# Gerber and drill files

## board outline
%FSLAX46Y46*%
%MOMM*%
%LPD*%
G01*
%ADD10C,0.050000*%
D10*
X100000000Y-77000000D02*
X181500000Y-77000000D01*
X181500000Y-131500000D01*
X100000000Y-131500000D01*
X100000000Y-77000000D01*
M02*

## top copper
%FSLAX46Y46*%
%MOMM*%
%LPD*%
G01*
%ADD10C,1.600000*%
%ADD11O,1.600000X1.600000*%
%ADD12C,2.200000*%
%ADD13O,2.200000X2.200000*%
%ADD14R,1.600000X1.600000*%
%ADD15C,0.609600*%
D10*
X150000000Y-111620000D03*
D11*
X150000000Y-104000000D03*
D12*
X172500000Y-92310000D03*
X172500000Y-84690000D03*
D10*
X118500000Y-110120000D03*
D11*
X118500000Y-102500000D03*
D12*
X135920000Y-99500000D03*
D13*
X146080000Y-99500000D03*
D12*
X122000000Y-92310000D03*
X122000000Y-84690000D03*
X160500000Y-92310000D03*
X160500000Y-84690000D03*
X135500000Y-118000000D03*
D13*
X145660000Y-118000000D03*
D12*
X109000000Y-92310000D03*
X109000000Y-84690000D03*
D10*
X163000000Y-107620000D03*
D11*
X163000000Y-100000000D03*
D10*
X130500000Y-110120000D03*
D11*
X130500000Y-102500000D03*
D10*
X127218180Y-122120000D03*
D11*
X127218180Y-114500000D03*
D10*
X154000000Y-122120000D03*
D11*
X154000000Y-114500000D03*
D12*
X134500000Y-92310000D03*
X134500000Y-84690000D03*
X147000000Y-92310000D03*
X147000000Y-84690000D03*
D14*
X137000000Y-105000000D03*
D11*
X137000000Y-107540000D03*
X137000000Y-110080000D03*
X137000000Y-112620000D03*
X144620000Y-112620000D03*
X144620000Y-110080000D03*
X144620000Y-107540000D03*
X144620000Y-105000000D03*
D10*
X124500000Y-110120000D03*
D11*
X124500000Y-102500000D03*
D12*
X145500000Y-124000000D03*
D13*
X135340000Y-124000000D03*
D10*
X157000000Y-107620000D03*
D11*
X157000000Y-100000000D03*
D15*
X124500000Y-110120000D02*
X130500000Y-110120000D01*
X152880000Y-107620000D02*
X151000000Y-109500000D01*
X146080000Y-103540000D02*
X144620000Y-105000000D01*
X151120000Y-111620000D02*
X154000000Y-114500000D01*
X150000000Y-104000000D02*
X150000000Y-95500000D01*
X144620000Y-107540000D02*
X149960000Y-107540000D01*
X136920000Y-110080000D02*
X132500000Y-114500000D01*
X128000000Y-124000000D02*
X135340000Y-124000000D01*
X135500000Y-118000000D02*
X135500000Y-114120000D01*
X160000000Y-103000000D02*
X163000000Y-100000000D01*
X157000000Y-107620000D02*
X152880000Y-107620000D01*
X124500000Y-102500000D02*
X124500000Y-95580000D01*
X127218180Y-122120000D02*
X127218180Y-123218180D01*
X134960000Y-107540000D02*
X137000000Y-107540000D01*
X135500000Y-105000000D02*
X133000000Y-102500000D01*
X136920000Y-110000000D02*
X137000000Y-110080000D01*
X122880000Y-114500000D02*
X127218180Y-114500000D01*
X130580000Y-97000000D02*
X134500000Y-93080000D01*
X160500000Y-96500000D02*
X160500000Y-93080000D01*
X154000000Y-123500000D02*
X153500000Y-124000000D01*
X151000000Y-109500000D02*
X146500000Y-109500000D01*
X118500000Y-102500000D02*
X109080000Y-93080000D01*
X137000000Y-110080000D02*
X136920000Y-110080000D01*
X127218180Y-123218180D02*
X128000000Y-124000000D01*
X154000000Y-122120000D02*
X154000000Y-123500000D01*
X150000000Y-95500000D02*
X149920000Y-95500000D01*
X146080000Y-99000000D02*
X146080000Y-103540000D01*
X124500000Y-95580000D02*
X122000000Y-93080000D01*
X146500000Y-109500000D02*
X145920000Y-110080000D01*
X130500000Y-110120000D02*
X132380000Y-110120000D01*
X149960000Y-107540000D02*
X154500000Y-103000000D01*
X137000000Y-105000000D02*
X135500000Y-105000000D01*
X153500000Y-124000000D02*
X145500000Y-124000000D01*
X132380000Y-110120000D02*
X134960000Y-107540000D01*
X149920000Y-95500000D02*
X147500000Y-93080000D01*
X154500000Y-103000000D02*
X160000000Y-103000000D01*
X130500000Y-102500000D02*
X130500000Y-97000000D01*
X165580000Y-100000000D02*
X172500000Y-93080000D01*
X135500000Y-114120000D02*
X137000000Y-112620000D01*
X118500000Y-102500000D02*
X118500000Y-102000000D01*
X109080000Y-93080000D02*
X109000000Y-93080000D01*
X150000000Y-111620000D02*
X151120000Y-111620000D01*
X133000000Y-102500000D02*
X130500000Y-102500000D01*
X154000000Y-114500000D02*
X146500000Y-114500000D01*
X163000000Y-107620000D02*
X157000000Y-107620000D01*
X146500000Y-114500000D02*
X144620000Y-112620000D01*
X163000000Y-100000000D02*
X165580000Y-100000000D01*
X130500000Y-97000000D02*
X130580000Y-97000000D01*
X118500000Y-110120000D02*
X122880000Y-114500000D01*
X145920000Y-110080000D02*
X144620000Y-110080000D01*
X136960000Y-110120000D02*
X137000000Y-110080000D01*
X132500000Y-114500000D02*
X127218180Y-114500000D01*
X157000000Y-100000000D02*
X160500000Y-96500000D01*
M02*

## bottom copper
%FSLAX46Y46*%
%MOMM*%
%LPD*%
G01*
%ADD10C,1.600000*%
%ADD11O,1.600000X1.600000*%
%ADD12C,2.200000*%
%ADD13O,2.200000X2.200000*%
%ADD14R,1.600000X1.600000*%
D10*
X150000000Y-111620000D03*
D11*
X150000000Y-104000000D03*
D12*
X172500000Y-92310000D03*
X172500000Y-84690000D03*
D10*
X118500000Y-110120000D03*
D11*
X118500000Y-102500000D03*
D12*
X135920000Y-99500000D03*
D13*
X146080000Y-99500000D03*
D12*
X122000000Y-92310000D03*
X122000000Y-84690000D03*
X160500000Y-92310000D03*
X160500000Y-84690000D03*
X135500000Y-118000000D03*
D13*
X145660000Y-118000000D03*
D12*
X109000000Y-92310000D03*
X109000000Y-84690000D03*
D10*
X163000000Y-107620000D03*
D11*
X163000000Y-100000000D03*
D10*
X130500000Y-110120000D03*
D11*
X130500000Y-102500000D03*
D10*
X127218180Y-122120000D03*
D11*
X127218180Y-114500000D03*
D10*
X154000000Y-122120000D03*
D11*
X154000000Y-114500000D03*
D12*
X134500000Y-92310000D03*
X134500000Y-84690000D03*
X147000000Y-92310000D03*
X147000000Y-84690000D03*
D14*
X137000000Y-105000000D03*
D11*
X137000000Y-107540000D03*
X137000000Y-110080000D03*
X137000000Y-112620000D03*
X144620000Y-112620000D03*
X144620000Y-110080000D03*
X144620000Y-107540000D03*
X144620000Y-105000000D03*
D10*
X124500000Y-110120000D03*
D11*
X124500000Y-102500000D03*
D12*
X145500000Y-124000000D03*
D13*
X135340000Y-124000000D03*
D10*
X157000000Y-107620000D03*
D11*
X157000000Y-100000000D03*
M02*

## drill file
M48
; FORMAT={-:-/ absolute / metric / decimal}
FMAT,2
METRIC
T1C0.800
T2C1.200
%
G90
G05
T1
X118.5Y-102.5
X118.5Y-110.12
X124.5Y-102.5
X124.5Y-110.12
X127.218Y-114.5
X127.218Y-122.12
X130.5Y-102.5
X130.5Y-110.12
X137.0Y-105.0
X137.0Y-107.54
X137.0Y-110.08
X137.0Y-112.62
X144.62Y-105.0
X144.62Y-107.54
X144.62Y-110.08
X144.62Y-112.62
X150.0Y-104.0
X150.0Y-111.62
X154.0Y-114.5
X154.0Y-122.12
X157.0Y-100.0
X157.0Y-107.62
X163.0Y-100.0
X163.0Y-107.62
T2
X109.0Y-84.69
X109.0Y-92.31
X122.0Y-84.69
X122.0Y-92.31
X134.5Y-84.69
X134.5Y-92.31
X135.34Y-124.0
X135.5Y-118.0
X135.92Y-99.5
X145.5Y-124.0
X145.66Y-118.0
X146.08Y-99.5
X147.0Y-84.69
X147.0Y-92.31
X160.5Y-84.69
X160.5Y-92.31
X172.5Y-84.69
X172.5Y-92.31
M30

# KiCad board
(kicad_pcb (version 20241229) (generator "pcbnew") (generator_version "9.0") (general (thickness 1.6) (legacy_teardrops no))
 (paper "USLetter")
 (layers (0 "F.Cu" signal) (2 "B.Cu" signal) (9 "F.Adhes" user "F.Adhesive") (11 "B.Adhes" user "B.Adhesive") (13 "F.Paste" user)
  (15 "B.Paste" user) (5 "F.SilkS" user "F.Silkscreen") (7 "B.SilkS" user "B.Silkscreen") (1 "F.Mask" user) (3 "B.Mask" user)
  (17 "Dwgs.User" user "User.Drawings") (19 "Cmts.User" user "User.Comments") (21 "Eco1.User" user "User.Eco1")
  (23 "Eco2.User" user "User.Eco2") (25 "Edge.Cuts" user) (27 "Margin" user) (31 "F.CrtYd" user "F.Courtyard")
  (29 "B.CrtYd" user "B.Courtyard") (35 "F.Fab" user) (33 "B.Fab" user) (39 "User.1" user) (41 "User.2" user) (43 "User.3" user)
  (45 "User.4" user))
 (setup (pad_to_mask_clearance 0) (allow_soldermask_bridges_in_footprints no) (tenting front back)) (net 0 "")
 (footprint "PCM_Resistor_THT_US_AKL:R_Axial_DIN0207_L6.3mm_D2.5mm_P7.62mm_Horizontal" (layer "F.Cu") (at 150 111.62 90)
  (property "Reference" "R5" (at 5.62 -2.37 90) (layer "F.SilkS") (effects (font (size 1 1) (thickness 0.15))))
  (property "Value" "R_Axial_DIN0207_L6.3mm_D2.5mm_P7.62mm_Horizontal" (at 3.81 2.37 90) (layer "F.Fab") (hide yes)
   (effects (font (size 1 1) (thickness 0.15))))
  (pad "1" thru_hole circle (at 0 0 90) (size 1.6 1.6) (drill 0.8) (layers "*.Cu" "*.Mask") (remove_unused_layers no))
  (pad "2" thru_hole oval (at 7.62 0 90) (size 1.6 1.6) (drill 0.8) (layers "*.Cu" "*.Mask") (remove_unused_layers no)))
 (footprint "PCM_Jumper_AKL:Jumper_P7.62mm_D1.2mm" (layer "F.Cu") (at 172.5 92.31 90)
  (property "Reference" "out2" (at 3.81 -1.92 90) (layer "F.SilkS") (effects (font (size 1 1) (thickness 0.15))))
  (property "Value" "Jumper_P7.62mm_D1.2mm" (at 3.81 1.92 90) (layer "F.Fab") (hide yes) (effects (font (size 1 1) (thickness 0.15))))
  (pad "1" thru_hole circle (at 0 0 90) (size 2.2 2.2) (drill 1.2) (layers "*.Cu" "*.Mask") (remove_unused_layers no))
  (pad "2" thru_hole circle (at 7.62 0 90) (size 2.2 2.2) (drill 1.2) (layers "*.Cu" "*.Mask") (remove_unused_layers no)))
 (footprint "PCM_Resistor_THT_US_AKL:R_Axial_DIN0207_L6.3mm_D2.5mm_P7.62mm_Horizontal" (layer "F.Cu") (at 118.5 110.12 90)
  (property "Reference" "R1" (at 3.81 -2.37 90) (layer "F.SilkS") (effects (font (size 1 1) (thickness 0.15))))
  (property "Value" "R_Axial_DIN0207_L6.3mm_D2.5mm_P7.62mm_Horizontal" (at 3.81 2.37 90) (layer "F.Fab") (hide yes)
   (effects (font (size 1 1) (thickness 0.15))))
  (pad "1" thru_hole circle (at 0 0 90) (size 1.6 1.6) (drill 0.8) (layers "*.Cu" "*.Mask") (remove_unused_layers no))
  (pad "2" thru_hole oval (at 7.62 0 90) (size 1.6 1.6) (drill 0.8) (layers "*.Cu" "*.Mask") (remove_unused_layers no)))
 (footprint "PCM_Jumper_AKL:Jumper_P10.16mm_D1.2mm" (layer "F.Cu") (at 135.92 99.5)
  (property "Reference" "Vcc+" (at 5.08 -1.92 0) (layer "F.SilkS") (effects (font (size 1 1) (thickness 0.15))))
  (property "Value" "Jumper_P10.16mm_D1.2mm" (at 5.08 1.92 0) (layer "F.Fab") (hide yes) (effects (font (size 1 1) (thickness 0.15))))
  (pad "1" thru_hole circle (at 0 0) (size 2.2 2.2) (drill 1.2) (layers "*.Cu" "*.Mask") (remove_unused_layers no))
  (pad "2" thru_hole oval (at 10.16 0) (size 2.2 2.2) (drill 1.2) (layers "*.Cu" "*.Mask") (remove_unused_layers no)))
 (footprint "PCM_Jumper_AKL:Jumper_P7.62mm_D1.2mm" (layer "F.Cu") (at 122 92.31 90)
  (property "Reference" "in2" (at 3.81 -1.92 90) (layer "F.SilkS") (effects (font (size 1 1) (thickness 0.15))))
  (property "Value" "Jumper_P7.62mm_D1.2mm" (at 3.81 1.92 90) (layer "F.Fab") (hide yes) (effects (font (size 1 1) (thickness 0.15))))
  (pad "1" thru_hole circle (at 0 0 90) (size 2.2 2.2) (drill 1.2) (layers "*.Cu" "*.Mask") (remove_unused_layers no))
  (pad "2" thru_hole circle (at 7.62 0 90) (size 2.2 2.2) (drill 1.2) (layers "*.Cu" "*.Mask") (remove_unused_layers no)))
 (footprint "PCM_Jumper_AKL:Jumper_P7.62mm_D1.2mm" (layer "F.Cu") (at 160.5 92.31 90)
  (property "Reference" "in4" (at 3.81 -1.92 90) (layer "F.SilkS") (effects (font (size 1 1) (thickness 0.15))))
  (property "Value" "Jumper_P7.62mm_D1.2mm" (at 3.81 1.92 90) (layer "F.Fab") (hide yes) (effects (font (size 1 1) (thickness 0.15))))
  (pad "1" thru_hole circle (at 0 0 90) (size 2.2 2.2) (drill 1.2) (layers "*.Cu" "*.Mask") (remove_unused_layers no))
  (pad "2" thru_hole circle (at 7.62 0 90) (size 2.2 2.2) (drill 1.2) (layers "*.Cu" "*.Mask") (remove_unused_layers no)))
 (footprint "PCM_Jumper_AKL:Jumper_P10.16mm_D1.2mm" (layer "F.Cu") (at 135.5 118)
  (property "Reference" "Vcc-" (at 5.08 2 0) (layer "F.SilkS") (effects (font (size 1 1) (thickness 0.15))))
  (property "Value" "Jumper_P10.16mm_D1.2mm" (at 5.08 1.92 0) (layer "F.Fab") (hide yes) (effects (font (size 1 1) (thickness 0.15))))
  (pad "1" thru_hole circle (at 0 0) (size 2.2 2.2) (drill 1.2) (layers "*.Cu" "*.Mask") (remove_unused_layers no))
  (pad "2" thru_hole oval (at 10.16 0) (size 2.2 2.2) (drill 1.2) (layers "*.Cu" "*.Mask") (remove_unused_layers no)))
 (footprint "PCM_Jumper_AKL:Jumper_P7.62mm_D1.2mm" (layer "F.Cu") (at 109 92.31 90)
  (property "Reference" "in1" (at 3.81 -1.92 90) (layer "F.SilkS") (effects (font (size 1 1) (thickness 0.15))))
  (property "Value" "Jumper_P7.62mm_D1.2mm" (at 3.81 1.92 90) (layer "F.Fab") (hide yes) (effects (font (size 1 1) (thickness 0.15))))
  (pad "1" thru_hole circle (at 0 0 90) (size 2.2 2.2) (drill 1.2) (layers "*.Cu" "*.Mask") (remove_unused_layers no))
  (pad "2" thru_hole circle (at 7.62 0 90) (size 2.2 2.2) (drill 1.2) (layers "*.Cu" "*.Mask") (remove_unused_layers no)))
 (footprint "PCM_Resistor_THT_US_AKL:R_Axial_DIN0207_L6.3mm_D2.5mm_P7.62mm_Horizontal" (layer "F.Cu") (at 163 107.62 90)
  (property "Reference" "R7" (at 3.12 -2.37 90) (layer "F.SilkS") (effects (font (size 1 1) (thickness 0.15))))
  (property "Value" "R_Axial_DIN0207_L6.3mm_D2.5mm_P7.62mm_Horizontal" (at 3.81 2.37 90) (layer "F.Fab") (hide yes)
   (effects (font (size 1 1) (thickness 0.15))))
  (pad "1" thru_hole circle (at 0 0 90) (size 1.6 1.6) (drill 0.8) (layers "*.Cu" "*.Mask") (remove_unused_layers no))
  (pad "2" thru_hole oval (at 7.62 0 90) (size 1.6 1.6) (drill 0.8) (layers "*.Cu" "*.Mask") (remove_unused_layers no)))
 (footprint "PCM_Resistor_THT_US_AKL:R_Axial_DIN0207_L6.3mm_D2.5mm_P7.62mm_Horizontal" (layer "F.Cu") (at 130.5 110.12 90)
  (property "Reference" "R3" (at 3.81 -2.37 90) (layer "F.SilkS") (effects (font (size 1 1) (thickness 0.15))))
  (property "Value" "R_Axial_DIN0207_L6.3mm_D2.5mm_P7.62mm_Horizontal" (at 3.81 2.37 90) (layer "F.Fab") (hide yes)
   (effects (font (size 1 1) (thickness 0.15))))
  (pad "1" thru_hole circle (at 0 0 90) (size 1.6 1.6) (drill 0.8) (layers "*.Cu" "*.Mask") (remove_unused_layers no))
  (pad "2" thru_hole oval (at 7.62 0 90) (size 1.6 1.6) (drill 0.8) (layers "*.Cu" "*.Mask") (remove_unused_layers no)))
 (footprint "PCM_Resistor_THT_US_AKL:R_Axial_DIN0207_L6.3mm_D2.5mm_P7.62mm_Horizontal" (layer "F.Cu") (at 127.21818 122.12 90)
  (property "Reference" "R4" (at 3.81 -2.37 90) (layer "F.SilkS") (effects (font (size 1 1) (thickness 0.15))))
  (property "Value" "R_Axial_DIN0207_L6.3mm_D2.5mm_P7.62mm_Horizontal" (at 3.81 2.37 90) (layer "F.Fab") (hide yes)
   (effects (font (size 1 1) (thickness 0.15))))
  (pad "1" thru_hole circle (at 0 0 90) (size 1.6 1.6) (drill 0.8) (layers "*.Cu" "*.Mask") (remove_unused_layers no))
  (pad "2" thru_hole oval (at 7.62 0 90) (size 1.6 1.6) (drill 0.8) (layers "*.Cu" "*.Mask") (remove_unused_layers no)))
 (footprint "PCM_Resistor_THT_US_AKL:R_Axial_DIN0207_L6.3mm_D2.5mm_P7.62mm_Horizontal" (layer "F.Cu") (at 154 122.12 90)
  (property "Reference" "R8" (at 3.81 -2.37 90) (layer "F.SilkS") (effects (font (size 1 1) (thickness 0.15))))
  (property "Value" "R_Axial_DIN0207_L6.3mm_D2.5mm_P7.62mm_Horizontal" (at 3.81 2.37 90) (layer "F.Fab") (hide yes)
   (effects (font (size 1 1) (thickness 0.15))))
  (pad "1" thru_hole circle (at 0 0 90) (size 1.6 1.6) (drill 0.8) (layers "*.Cu" "*.Mask") (remove_unused_layers no))
  (pad "2" thru_hole oval (at 7.62 0 90) (size 1.6 1.6) (drill 0.8) (layers "*.Cu" "*.Mask") (remove_unused_layers no)))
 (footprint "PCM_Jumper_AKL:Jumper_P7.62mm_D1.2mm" (layer "F.Cu") (at 134.5 92.31 90)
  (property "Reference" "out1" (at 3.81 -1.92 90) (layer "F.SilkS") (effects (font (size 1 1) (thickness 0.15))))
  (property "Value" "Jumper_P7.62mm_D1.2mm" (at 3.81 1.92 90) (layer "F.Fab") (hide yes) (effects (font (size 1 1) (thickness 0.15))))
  (pad "1" thru_hole circle (at 0 0 90) (size 2.2 2.2) (drill 1.2) (layers "*.Cu" "*.Mask") (remove_unused_layers no))
  (pad "2" thru_hole circle (at 7.62 0 90) (size 2.2 2.2) (drill 1.2) (layers "*.Cu" "*.Mask") (remove_unused_layers no)))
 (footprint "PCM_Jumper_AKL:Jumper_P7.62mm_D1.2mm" (layer "F.Cu") (at 147 92.31 90)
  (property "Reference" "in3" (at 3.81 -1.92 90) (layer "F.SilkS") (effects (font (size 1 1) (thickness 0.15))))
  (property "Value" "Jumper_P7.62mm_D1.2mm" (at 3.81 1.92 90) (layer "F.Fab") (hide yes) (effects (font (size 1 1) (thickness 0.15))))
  (pad "1" thru_hole circle (at 0 0 90) (size 2.2 2.2) (drill 1.2) (layers "*.Cu" "*.Mask") (remove_unused_layers no))
  (pad "2" thru_hole circle (at 7.62 0 90) (size 2.2 2.2) (drill 1.2) (layers "*.Cu" "*.Mask") (remove_unused_layers no)))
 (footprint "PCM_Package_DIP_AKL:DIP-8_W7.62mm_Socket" (layer "F.Cu") (at 137 105)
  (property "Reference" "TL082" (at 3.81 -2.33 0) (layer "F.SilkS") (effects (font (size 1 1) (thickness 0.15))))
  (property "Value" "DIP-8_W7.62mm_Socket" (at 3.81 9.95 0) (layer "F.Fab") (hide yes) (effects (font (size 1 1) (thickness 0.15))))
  (pad "1" thru_hole rect (at 0 0) (size 1.6 1.6) (drill 0.8) (layers "*.Cu" "*.Mask") (remove_unused_layers no))
  (pad "2" thru_hole oval (at 0 2.54) (size 1.6 1.6) (drill 0.8) (layers "*.Cu" "*.Mask") (remove_unused_layers no))
  (pad "3" thru_hole oval (at 0 5.08) (size 1.6 1.6) (drill 0.8) (layers "*.Cu" "*.Mask") (remove_unused_layers no))
  (pad "4" thru_hole oval (at 0 7.62) (size 1.6 1.6) (drill 0.8) (layers "*.Cu" "*.Mask") (remove_unused_layers no))
  (pad "5" thru_hole oval (at 7.62 7.62) (size 1.6 1.6) (drill 0.8) (layers "*.Cu" "*.Mask") (remove_unused_layers no))
  (pad "6" thru_hole oval (at 7.62 5.08) (size 1.6 1.6) (drill 0.8) (layers "*.Cu" "*.Mask") (remove_unused_layers no))
  (pad "7" thru_hole oval (at 7.62 2.54) (size 1.6 1.6) (drill 0.8) (layers "*.Cu" "*.Mask") (remove_unused_layers no))
  (pad "8" thru_hole oval (at 7.62 0) (size 1.6 1.6) (drill 0.8) (layers "*.Cu" "*.Mask") (remove_unused_layers no)))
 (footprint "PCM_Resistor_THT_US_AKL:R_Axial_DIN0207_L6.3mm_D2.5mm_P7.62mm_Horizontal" (layer "F.Cu") (at 124.5 110.12 90)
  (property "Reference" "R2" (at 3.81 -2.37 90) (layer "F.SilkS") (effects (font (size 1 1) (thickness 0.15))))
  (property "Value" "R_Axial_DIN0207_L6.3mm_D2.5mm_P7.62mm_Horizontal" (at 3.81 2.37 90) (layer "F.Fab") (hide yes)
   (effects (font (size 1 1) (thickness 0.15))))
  (pad "1" thru_hole circle (at 0 0 90) (size 1.6 1.6) (drill 0.8) (layers "*.Cu" "*.Mask") (remove_unused_layers no))
  (pad "2" thru_hole oval (at 7.62 0 90) (size 1.6 1.6) (drill 0.8) (layers "*.Cu" "*.Mask") (remove_unused_layers no)))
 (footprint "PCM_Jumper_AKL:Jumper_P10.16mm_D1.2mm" (layer "F.Cu") (at 145.5 124 180)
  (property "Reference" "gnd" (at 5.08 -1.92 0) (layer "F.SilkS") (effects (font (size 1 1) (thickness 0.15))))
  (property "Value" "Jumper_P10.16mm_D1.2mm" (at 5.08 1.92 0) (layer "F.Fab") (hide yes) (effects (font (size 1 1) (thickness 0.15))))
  (pad "1" thru_hole circle (at 0 0 180) (size 2.2 2.2) (drill 1.2) (layers "*.Cu" "*.Mask") (remove_unused_layers no))
  (pad "2" thru_hole oval (at 10.16 0 180) (size 2.2 2.2) (drill 1.2) (layers "*.Cu" "*.Mask") (remove_unused_layers no)))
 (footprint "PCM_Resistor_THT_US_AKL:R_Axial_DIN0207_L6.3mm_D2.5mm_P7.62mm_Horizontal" (layer "F.Cu") (at 157 107.62 90)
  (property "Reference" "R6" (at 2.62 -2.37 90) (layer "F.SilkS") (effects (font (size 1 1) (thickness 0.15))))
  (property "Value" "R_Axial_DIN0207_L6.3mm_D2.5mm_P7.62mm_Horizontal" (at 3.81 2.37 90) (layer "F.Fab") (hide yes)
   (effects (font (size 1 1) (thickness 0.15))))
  (pad "1" thru_hole circle (at 0 0 90) (size 1.6 1.6) (drill 0.8) (layers "*.Cu" "*.Mask") (remove_unused_layers no))
  (pad "2" thru_hole oval (at 7.62 0 90) (size 1.6 1.6) (drill 0.8) (layers "*.Cu" "*.Mask") (remove_unused_layers no)))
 (gr_rect (start 100 77) (end 181.5 131.5) (stroke (width 0.05) (type default)) (fill no) (layer "Edge.Cuts"))
 (segment (start 124.5 110.12) (end 130.5 110.12) (width 0.6096) (layer "F.Cu") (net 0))
 (segment (start 152.88 107.62) (end 151 109.5) (width 0.6096) (layer "F.Cu") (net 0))
 (segment (start 146.08 103.54) (end 144.62 105) (width 0.6096) (layer "F.Cu") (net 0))
 (segment (start 151.12 111.62) (end 154 114.5) (width 0.6096) (layer "F.Cu") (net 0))
 (segment (start 150 104) (end 150 95.5) (width 0.6096) (layer "F.Cu") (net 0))
 (segment (start 144.62 107.54) (end 149.96 107.54) (width 0.6096) (layer "F.Cu") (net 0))
 (segment (start 136.92 110.08) (end 132.5 114.5) (width 0.6096) (layer "F.Cu") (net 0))
 (segment (start 128 124) (end 135.34 124) (width 0.6096) (layer "F.Cu") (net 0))
 (segment (start 135.5 118) (end 135.5 114.12) (width 0.6096) (layer "F.Cu") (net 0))
 (segment (start 160 103) (end 163 100) (width 0.6096) (layer "F.Cu") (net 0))
 (segment (start 157 107.62) (end 152.88 107.62) (width 0.6096) (layer "F.Cu") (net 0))
 (segment (start 124.5 102.5) (end 124.5 95.58) (width 0.6096) (layer "F.Cu") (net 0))
 (segment (start 127.21818 122.12) (end 127.21818 123.21818) (width 0.6096) (layer "F.Cu") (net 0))
 (segment (start 134.96 107.54) (end 137 107.54) (width 0.6096) (layer "F.Cu") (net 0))
 (segment (start 135.5 105) (end 133 102.5) (width 0.6096) (layer "F.Cu") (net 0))
 (segment (start 136.92 110) (end 137 110.08) (width 0.6096) (layer "F.Cu") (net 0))
 (segment (start 122.88 114.5) (end 127.21818 114.5) (width 0.6096) (layer "F.Cu") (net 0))
 (segment (start 130.58 97) (end 134.5 93.08) (width 0.6096) (layer "F.Cu") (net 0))
 (segment (start 160.5 96.5) (end 160.5 93.08) (width 0.6096) (layer "F.Cu") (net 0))
 (segment (start 154 123.5) (end 153.5 124) (width 0.6096) (layer "F.Cu") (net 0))
 (segment (start 151 109.5) (end 146.5 109.5) (width 0.6096) (layer "F.Cu") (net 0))
 (segment (start 118.5 102.5) (end 109.08 93.08) (width 0.6096) (layer "F.Cu") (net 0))
 (segment (start 137 110.08) (end 136.92 110.08) (width 0.6096) (layer "F.Cu") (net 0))
 (segment (start 127.21818 123.21818) (end 128 124) (width 0.6096) (layer "F.Cu") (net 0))
 (segment (start 154 122.12) (end 154 123.5) (width 0.6096) (layer "F.Cu") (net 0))
 (segment (start 150 95.5) (end 149.92 95.5) (width 0.6096) (layer "F.Cu") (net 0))
 (segment (start 146.08 99) (end 146.08 103.54) (width 0.6096) (layer "F.Cu") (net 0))
 (segment (start 124.5 95.58) (end 122 93.08) (width 0.6096) (layer "F.Cu") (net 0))
 (segment (start 146.5 109.5) (end 145.92 110.08) (width 0.6096) (layer "F.Cu") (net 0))
 (segment (start 130.5 110.12) (end 132.38 110.12) (width 0.6096) (layer "F.Cu") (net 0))
 (segment (start 149.96 107.54) (end 154.5 103) (width 0.6096) (layer "F.Cu") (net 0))
 (segment (start 137 105) (end 135.5 105) (width 0.6096) (layer "F.Cu") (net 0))
 (segment (start 153.5 124) (end 145.5 124) (width 0.6096) (layer "F.Cu") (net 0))
 (segment (start 132.38 110.12) (end 134.96 107.54) (width 0.6096) (layer "F.Cu") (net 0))
 (segment (start 149.92 95.5) (end 147.5 93.08) (width 0.6096) (layer "F.Cu") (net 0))
 (segment (start 154.5 103) (end 160 103) (width 0.6096) (layer "F.Cu") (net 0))
 (segment (start 130.5 102.5) (end 130.5 97) (width 0.6096) (layer "F.Cu") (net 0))
 (segment (start 165.58 100) (end 172.5 93.08) (width 0.6096) (layer "F.Cu") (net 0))
 (segment (start 135.5 114.12) (end 137 112.62) (width 0.6096) (layer "F.Cu") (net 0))
 (segment (start 118.5 102.5) (end 118.5 102) (width 0.6096) (layer "F.Cu") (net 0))
 (segment (start 109.08 93.08) (end 109 93.08) (width 0.6096) (layer "F.Cu") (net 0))
 (segment (start 150 111.62) (end 151.12 111.62) (width 0.6096) (layer "F.Cu") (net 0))
 (segment (start 133 102.5) (end 130.5 102.5) (width 0.6096) (layer "F.Cu") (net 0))
 (segment (start 154 114.5) (end 146.5 114.5) (width 0.6096) (layer "F.Cu") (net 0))
 (segment (start 163 107.62) (end 157 107.62) (width 0.6096) (layer "F.Cu") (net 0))
 (segment (start 146.5 114.5) (end 144.62 112.62) (width 0.6096) (layer "F.Cu") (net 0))
 (segment (start 163 100) (end 165.58 100) (width 0.6096) (layer "F.Cu") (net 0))
 (segment (start 130.5 97) (end 130.58 97) (width 0.6096) (layer "F.Cu") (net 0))
 (segment (start 118.5 110.12) (end 122.88 114.5) (width 0.6096) (layer "F.Cu") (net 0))
 (segment (start 145.92 110.08) (end 144.62 110.08) (width 0.6096) (layer "F.Cu") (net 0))
 (segment (start 136.96 110.12) (end 137 110.08) (width 0.6096) (layer "F.Cu") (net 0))
 (segment (start 132.5 114.5) (end 127.21818 114.5) (width 0.6096) (layer "F.Cu") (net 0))
 (segment (start 157 100) (end 160.5 96.5) (width 0.6096) (layer "F.Cu") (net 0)))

